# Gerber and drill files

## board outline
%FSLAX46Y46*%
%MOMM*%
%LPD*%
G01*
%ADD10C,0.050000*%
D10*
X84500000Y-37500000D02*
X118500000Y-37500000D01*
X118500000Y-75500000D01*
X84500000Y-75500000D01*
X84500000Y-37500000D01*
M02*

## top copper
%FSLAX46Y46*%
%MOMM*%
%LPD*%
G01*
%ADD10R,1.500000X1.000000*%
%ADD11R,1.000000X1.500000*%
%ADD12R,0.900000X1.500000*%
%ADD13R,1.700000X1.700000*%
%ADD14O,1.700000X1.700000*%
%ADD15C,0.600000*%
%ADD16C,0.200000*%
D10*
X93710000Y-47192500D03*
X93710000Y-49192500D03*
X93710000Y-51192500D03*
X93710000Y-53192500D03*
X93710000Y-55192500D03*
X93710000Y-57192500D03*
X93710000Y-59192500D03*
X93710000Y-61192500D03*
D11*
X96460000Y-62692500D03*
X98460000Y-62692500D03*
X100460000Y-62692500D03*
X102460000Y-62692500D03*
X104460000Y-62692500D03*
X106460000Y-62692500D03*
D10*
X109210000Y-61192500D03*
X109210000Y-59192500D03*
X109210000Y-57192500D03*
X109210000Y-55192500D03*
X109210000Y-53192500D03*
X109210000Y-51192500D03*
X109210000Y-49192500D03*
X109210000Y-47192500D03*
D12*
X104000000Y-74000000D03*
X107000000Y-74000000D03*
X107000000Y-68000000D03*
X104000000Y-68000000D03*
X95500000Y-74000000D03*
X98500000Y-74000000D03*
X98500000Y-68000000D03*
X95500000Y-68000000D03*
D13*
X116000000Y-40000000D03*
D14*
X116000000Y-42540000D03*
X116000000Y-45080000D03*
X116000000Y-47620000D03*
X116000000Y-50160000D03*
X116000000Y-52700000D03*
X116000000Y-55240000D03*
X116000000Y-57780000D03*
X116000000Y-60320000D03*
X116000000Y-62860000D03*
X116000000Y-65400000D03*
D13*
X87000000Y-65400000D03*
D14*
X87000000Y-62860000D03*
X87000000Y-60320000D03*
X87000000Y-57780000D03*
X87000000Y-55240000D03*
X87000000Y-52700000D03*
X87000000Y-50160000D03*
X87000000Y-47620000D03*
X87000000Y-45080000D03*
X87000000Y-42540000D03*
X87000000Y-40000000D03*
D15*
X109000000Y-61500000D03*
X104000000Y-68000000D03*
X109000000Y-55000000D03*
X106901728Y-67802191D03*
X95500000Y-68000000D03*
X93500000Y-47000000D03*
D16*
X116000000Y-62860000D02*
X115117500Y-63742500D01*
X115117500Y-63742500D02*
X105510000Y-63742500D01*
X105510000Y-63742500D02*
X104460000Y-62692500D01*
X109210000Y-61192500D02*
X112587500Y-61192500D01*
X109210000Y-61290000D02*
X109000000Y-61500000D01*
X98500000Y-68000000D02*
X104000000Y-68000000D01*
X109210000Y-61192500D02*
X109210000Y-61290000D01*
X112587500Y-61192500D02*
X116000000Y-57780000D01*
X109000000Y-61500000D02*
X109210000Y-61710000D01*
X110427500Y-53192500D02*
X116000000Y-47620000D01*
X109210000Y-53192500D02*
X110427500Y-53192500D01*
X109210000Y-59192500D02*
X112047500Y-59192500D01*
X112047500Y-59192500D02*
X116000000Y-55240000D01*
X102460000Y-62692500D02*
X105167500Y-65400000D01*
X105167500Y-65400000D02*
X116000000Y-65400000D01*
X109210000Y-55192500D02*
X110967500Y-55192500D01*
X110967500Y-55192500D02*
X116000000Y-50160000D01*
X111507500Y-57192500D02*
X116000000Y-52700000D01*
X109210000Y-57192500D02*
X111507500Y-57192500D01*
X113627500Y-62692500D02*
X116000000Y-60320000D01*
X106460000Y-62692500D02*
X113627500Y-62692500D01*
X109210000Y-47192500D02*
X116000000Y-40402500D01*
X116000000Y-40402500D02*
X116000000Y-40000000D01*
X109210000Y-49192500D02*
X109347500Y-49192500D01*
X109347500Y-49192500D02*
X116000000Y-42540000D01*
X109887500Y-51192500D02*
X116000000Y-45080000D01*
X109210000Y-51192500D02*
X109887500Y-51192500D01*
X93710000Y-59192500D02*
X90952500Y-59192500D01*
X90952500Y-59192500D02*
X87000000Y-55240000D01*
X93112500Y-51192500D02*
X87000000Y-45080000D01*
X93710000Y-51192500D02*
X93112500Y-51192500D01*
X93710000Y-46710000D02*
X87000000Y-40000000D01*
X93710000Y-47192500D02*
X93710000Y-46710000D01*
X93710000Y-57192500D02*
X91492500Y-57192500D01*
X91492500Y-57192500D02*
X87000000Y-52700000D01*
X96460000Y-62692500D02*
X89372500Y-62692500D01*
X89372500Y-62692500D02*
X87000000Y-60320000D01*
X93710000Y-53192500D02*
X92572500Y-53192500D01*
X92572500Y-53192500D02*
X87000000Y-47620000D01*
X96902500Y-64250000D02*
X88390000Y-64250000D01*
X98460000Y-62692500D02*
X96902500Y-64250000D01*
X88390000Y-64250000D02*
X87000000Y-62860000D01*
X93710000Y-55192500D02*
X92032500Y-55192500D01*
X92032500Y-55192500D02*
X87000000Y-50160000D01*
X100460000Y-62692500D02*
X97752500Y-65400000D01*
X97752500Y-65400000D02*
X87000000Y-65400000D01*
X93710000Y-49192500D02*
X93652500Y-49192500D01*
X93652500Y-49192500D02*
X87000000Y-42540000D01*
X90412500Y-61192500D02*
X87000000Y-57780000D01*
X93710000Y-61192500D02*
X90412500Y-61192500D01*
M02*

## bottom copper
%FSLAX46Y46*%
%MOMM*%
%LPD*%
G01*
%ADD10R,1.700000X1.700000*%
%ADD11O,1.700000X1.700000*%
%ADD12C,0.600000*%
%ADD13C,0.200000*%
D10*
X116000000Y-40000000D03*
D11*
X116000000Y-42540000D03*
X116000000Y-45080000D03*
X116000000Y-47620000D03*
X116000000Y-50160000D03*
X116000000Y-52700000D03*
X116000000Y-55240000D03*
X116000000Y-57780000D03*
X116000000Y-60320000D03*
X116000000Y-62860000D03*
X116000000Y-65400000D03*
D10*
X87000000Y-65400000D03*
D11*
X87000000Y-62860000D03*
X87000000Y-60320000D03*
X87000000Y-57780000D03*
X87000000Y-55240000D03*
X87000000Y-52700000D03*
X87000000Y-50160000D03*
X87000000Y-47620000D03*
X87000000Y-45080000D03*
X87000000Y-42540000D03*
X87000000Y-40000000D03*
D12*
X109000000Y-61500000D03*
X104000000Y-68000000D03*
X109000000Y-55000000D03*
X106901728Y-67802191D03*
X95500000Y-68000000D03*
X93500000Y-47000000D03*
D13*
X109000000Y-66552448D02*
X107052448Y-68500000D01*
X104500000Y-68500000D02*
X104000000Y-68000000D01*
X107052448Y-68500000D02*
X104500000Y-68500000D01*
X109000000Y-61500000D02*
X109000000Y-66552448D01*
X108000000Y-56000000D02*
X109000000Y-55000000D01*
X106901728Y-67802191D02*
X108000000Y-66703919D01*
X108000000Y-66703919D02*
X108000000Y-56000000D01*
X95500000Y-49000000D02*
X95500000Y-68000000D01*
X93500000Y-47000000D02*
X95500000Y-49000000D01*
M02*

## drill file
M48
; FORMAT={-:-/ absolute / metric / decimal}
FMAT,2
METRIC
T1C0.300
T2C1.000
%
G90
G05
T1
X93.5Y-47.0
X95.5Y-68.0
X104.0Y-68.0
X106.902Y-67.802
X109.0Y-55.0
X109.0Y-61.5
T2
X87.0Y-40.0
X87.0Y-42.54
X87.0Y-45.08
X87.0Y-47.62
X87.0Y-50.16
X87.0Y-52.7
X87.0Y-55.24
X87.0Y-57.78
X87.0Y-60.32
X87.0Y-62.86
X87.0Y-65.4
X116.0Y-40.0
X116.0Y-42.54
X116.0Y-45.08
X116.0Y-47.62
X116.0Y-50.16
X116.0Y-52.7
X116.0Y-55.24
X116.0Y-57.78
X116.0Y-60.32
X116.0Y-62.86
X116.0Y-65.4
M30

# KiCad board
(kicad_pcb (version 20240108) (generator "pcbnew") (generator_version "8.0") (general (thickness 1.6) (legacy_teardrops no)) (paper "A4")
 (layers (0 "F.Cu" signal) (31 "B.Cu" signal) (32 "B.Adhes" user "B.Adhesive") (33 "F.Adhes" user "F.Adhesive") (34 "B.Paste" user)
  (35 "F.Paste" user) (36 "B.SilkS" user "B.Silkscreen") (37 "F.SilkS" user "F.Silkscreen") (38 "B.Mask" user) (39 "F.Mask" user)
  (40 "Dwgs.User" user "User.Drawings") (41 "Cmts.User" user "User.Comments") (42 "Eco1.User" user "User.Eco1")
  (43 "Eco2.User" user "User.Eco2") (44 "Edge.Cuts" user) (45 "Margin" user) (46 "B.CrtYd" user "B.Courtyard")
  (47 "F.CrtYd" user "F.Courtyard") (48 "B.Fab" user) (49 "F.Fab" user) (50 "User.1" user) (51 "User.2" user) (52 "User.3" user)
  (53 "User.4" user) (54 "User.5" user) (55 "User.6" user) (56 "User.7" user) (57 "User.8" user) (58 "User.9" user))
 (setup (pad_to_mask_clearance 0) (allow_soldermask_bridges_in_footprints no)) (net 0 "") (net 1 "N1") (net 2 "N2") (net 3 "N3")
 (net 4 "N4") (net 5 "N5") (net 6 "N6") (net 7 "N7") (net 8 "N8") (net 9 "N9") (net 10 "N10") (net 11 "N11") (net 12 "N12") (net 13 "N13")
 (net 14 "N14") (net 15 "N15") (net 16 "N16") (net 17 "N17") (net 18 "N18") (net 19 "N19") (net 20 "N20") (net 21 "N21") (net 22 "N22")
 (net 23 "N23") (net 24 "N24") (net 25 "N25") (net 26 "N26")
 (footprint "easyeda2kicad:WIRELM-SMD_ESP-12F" (layer "F.Cu") (at 101.46 54.9425)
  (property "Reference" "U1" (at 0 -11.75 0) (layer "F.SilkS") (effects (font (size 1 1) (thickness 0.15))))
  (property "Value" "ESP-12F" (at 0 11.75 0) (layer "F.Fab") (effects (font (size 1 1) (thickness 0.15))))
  (pad "1" smd rect (at -7.75 -7.75) (size 1.5 1) (layers "F.Cu" "F.Paste" "F.Mask") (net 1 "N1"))
  (pad "2" smd rect (at -7.75 -5.75) (size 1.5 1) (layers "F.Cu" "F.Paste" "F.Mask") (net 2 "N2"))
  (pad "3" smd rect (at -7.75 -3.75) (size 1.5 1) (layers "F.Cu" "F.Paste" "F.Mask") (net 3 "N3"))
  (pad "4" smd rect (at -7.75 -1.75) (size 1.5 1) (layers "F.Cu" "F.Paste" "F.Mask") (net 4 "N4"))
  (pad "5" smd rect (at -7.75 0.25) (size 1.5 1) (layers "F.Cu" "F.Paste" "F.Mask") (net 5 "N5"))
  (pad "6" smd rect (at -7.75 2.25) (size 1.5 1) (layers "F.Cu" "F.Paste" "F.Mask") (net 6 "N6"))
  (pad "7" smd rect (at -7.75 4.25) (size 1.5 1) (layers "F.Cu" "F.Paste" "F.Mask") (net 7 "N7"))
  (pad "8" smd rect (at -7.75 6.25) (size 1.5 1) (layers "F.Cu" "F.Paste" "F.Mask") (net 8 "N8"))
  (pad "9" smd rect (at -5 7.75 90) (size 1.5 1) (layers "F.Cu" "F.Paste" "F.Mask") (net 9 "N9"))
  (pad "10" smd rect (at -3 7.75 90) (size 1.5 1) (layers "F.Cu" "F.Paste" "F.Mask") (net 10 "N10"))
  (pad "11" smd rect (at -1 7.75 90) (size 1.5 1) (layers "F.Cu" "F.Paste" "F.Mask") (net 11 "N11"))
  (pad "12" smd rect (at 1 7.75 90) (size 1.5 1) (layers "F.Cu" "F.Paste" "F.Mask") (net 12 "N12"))
  (pad "13" smd rect (at 3 7.75 90) (size 1.5 1) (layers "F.Cu" "F.Paste" "F.Mask") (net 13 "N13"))
  (pad "14" smd rect (at 5 7.75 90) (size 1.5 1) (layers "F.Cu" "F.Paste" "F.Mask") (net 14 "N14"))
  (pad "15" smd rect (at 7.75 6.25 180) (size 1.5 1) (layers "F.Cu" "F.Paste" "F.Mask") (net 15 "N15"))
  (pad "16" smd rect (at 7.75 4.25 180) (size 1.5 1) (layers "F.Cu" "F.Paste" "F.Mask") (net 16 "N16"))
  (pad "17" smd rect (at 7.75 2.25 180) (size 1.5 1) (layers "F.Cu" "F.Paste" "F.Mask") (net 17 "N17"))
  (pad "18" smd rect (at 7.75 0.25 180) (size 1.5 1) (layers "F.Cu" "F.Paste" "F.Mask") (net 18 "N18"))
  (pad "19" smd rect (at 7.75 -1.75 180) (size 1.5 1) (layers "F.Cu" "F.Paste" "F.Mask") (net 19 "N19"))
  (pad "20" smd rect (at 7.75 -3.75 180) (size 1.5 1) (layers "F.Cu" "F.Paste" "F.Mask") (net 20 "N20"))
  (pad "21" smd rect (at 7.75 -5.75 180) (size 1.5 1) (layers "F.Cu" "F.Paste" "F.Mask") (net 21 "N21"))
  (pad "22" smd rect (at 7.75 -7.75 180) (size 1.5 1) (layers "F.Cu" "F.Paste" "F.Mask") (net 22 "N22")))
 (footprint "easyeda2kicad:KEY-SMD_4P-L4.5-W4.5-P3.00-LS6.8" (layer "F.Cu") (at 105.5 71 90)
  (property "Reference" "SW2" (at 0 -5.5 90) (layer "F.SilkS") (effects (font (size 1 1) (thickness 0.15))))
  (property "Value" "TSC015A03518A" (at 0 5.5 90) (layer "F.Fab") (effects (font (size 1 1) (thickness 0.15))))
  (pad "1" smd rect (at -3 -1.5 90) (size 1.5 0.9) (layers "F.Cu" "F.Paste" "F.Mask") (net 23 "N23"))
  (pad "2" smd rect (at -3 1.5 90) (size 1.5 0.9) (layers "F.Cu" "F.Paste" "F.Mask") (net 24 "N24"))
  (pad "3" smd rect (at 3 1.5 90) (size 1.5 0.9) (layers "F.Cu" "F.Paste" "F.Mask") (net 18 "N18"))
  (pad "4" smd rect (at 3 -1.5 90) (size 1.5 0.9) (layers "F.Cu" "F.Paste" "F.Mask") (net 15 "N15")))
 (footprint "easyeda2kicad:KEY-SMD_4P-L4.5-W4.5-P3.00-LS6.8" (layer "F.Cu") (at 97 71 90)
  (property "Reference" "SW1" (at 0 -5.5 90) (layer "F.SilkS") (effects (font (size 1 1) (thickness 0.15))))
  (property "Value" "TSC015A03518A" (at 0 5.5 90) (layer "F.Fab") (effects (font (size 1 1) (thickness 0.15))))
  (pad "1" smd rect (at -3 -1.5 90) (size 1.5 0.9) (layers "F.Cu" "F.Paste" "F.Mask") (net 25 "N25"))
  (pad "2" smd rect (at -3 1.5 90) (size 1.5 0.9) (layers "F.Cu" "F.Paste" "F.Mask") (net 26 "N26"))
  (pad "3" smd rect (at 3 1.5 90) (size 1.5 0.9) (layers "F.Cu" "F.Paste" "F.Mask") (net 15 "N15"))
  (pad "4" smd rect (at 3 -1.5 90) (size 1.5 0.9) (layers "F.Cu" "F.Paste" "F.Mask") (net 1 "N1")))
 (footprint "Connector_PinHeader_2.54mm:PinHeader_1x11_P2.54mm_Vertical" (layer "B.Cu") (at 116 40 180)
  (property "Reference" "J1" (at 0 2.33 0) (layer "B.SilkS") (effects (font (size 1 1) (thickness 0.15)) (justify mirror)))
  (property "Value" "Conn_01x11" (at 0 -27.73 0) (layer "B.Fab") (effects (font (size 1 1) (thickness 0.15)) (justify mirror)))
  (pad "1" thru_hole rect (at 0 0 180) (size 1.7 1.7) (drill 1) (layers "*.Cu" "*.Mask") (remove_unused_layers no) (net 22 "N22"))
  (pad "2" thru_hole oval (at 0 -2.54 180) (size 1.7 1.7) (drill 1) (layers "*.Cu" "*.Mask") (remove_unused_layers no) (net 21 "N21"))
  (pad "3" thru_hole oval (at 0 -5.08 180) (size 1.7 1.7) (drill 1) (layers "*.Cu" "*.Mask") (remove_unused_layers no) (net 20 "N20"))
  (pad "4" thru_hole oval (at 0 -7.62 180) (size 1.7 1.7) (drill 1) (layers "*.Cu" "*.Mask") (remove_unused_layers no) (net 19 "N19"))
  (pad "5" thru_hole oval (at 0 -10.16 180) (size 1.7 1.7) (drill 1) (layers "*.Cu" "*.Mask") (remove_unused_layers no) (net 18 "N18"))
  (pad "6" thru_hole oval (at 0 -12.7 180) (size 1.7 1.7) (drill 1) (layers "*.Cu" "*.Mask") (remove_unused_layers no) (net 17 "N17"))
  (pad "7" thru_hole oval (at 0 -15.24 180) (size 1.7 1.7) (drill 1) (layers "*.Cu" "*.Mask") (remove_unused_layers no) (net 16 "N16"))
  (pad "8" thru_hole oval (at 0 -17.78 180) (size 1.7 1.7) (drill 1) (layers "*.Cu" "*.Mask") (remove_unused_layers no) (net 15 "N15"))
  (pad "9" thru_hole oval (at 0 -20.32 180) (size 1.7 1.7) (drill 1) (layers "*.Cu" "*.Mask") (remove_unused_layers no) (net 14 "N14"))
  (pad "10" thru_hole oval (at 0 -22.86 180) (size 1.7 1.7) (drill 1) (layers "*.Cu" "*.Mask") (remove_unused_layers no) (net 13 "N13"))
  (pad "11" thru_hole oval (at 0 -25.4 180) (size 1.7 1.7) (drill 1) (layers "*.Cu" "*.Mask") (remove_unused_layers no) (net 12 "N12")))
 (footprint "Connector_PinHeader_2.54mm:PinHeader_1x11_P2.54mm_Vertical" (layer "B.Cu") (at 87 65.4)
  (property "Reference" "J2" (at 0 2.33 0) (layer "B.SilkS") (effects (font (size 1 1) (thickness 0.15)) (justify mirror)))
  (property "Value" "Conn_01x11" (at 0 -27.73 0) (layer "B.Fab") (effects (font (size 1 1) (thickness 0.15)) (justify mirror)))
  (pad "1" thru_hole rect (at 0 0) (size 1.7 1.7) (drill 1) (layers "*.Cu" "*.Mask") (remove_unused_layers no) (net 11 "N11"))
  (pad "2" thru_hole oval (at 0 -2.54) (size 1.7 1.7) (drill 1) (layers "*.Cu" "*.Mask") (remove_unused_layers no) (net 10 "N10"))
  (pad "3" thru_hole oval (at 0 -5.08) (size 1.7 1.7) (drill 1) (layers "*.Cu" "*.Mask") (remove_unused_layers no) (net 9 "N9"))
  (pad "4" thru_hole oval (at 0 -7.62) (size 1.7 1.7) (drill 1) (layers "*.Cu" "*.Mask") (remove_unused_layers no) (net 8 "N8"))
  (pad "5" thru_hole oval (at 0 -10.16) (size 1.7 1.7) (drill 1) (layers "*.Cu" "*.Mask") (remove_unused_layers no) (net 7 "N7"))
  (pad "6" thru_hole oval (at 0 -12.7) (size 1.7 1.7) (drill 1) (layers "*.Cu" "*.Mask") (remove_unused_layers no) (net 6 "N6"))
  (pad "7" thru_hole oval (at 0 -15.24) (size 1.7 1.7) (drill 1) (layers "*.Cu" "*.Mask") (remove_unused_layers no) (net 5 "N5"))
  (pad "8" thru_hole oval (at 0 -17.78) (size 1.7 1.7) (drill 1) (layers "*.Cu" "*.Mask") (remove_unused_layers no) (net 4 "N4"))
  (pad "9" thru_hole oval (at 0 -20.32) (size 1.7 1.7) (drill 1) (layers "*.Cu" "*.Mask") (remove_unused_layers no) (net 3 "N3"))
  (pad "10" thru_hole oval (at 0 -22.86) (size 1.7 1.7) (drill 1) (layers "*.Cu" "*.Mask") (remove_unused_layers no) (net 2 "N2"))
  (pad "11" thru_hole oval (at 0 -25.4) (size 1.7 1.7) (drill 1) (layers "*.Cu" "*.Mask") (remove_unused_layers no) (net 1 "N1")))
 (gr_rect (start 84.5 37.5) (end 118.5 75.5) (stroke (width 0.05) (type default)) (fill none) (layer "Edge.Cuts"))
 (segment (start 116 62.86) (end 115.1175 63.7425) (width 0.2) (layer "F.Cu") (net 13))
 (segment (start 115.1175 63.7425) (end 105.51 63.7425) (width 0.2) (layer "F.Cu") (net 13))
 (segment (start 105.51 63.7425) (end 104.46 62.6925) (width 0.2) (layer "F.Cu") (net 13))
 (segment (start 109.21 61.1925) (end 112.5875 61.1925) (width 0.2) (layer "F.Cu") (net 15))
 (segment (start 109.21 61.29) (end 109 61.5) (width 0.2) (layer "F.Cu") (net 15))
 (segment (start 98.5 68) (end 104 68) (width 0.2) (layer "F.Cu") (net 15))
 (segment (start 109.21 61.1925) (end 109.21 61.29) (width 0.2) (layer "F.Cu") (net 15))
 (segment (start 112.5875 61.1925) (end 116 57.78) (width 0.2) (layer "F.Cu") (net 15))
 (segment (start 109 61.5) (end 109.21 61.71) (width 0.2) (layer "F.Cu") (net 15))
 (via (at 109 61.5) (size 0.6) (drill 0.3) (layers "F.Cu" "B.Cu") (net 15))
 (via (at 104 68) (size 0.6) (drill 0.3) (layers "F.Cu" "B.Cu") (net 15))
 (segment (start 109 66.552448) (end 107.052448 68.5) (width 0.2) (layer "B.Cu") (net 15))
 (segment (start 104.5 68.5) (end 104 68) (width 0.2) (layer "B.Cu") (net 15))
 (segment (start 107.052448 68.5) (end 104.5 68.5) (width 0.2) (layer "B.Cu") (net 15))
 (segment (start 109 61.5) (end 109 66.552448) (width 0.2) (layer "B.Cu") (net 15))
 (segment (start 110.4275 53.1925) (end 116 47.62) (width 0.2) (layer "F.Cu") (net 19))
 (segment (start 109.21 53.1925) (end 110.4275 53.1925) (width 0.2) (layer "F.Cu") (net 19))
 (segment (start 109.21 59.1925) (end 112.0475 59.1925) (width 0.2) (layer "F.Cu") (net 16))
 (segment (start 112.0475 59.1925) (end 116 55.24) (width 0.2) (layer "F.Cu") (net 16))
 (segment (start 102.46 62.6925) (end 105.1675 65.4) (width 0.2) (layer "F.Cu") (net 12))
 (segment (start 105.1675 65.4) (end 116 65.4) (width 0.2) (layer "F.Cu") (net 12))
 (segment (start 109.21 55.1925) (end 110.9675 55.1925) (width 0.2) (layer "F.Cu") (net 18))
 (segment (start 110.9675 55.1925) (end 116 50.16) (width 0.2) (layer "F.Cu") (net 18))
 (via (at 109 55) (size 0.6) (drill 0.3) (layers "F.Cu" "B.Cu") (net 18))
 (via (at 106.901728 67.802191) (size 0.6) (drill 0.3) (layers "F.Cu" "B.Cu") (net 18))
 (segment (start 108 56) (end 109 55) (width 0.2) (layer "B.Cu") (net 18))
 (segment (start 106.901728 67.802191) (end 108 66.703919) (width 0.2) (layer "B.Cu") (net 18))
 (segment (start 108 66.703919) (end 108 56) (width 0.2) (layer "B.Cu") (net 18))
 (segment (start 111.5075 57.1925) (end 116 52.7) (width 0.2) (layer "F.Cu") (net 17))
 (segment (start 109.21 57.1925) (end 111.5075 57.1925) (width 0.2) (layer "F.Cu") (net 17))
 (segment (start 113.6275 62.6925) (end 116 60.32) (width 0.2) (layer "F.Cu") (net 14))
 (segment (start 106.46 62.6925) (end 113.6275 62.6925) (width 0.2) (layer "F.Cu") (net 14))
 (segment (start 109.21 47.1925) (end 116 40.4025) (width 0.2) (layer "F.Cu") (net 22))
 (segment (start 116 40.4025) (end 116 40) (width 0.2) (layer "F.Cu") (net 22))
 (segment (start 109.21 49.1925) (end 109.3475 49.1925) (width 0.2) (layer "F.Cu") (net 21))
 (segment (start 109.3475 49.1925) (end 116 42.54) (width 0.2) (layer "F.Cu") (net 21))
 (segment (start 109.8875 51.1925) (end 116 45.08) (width 0.2) (layer "F.Cu") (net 20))
 (segment (start 109.21 51.1925) (end 109.8875 51.1925) (width 0.2) (layer "F.Cu") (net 20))
 (segment (start 93.71 59.1925) (end 90.9525 59.1925) (width 0.2) (layer "F.Cu") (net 7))
 (segment (start 90.9525 59.1925) (end 87 55.24) (width 0.2) (layer "F.Cu") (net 7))
 (segment (start 93.1125 51.1925) (end 87 45.08) (width 0.2) (layer "F.Cu") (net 3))
 (segment (start 93.71 51.1925) (end 93.1125 51.1925) (width 0.2) (layer "F.Cu") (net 3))
 (segment (start 93.71 46.71) (end 87 40) (width 0.2) (layer "F.Cu") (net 1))
 (segment (start 93.71 47.1925) (end 93.71 46.71) (width 0.2) (layer "F.Cu") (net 1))
 (via (at 95.5 68) (size 0.6) (drill 0.3) (layers "F.Cu" "B.Cu") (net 1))
 (via (at 93.5 47) (size 0.6) (drill 0.3) (layers "F.Cu" "B.Cu") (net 1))
 (segment (start 95.5 49) (end 95.5 68) (width 0.2) (layer "B.Cu") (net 1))
 (segment (start 93.5 47) (end 95.5 49) (width 0.2) (layer "B.Cu") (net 1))
 (segment (start 93.71 57.1925) (end 91.4925 57.1925) (width 0.2) (layer "F.Cu") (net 6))
 (segment (start 91.4925 57.1925) (end 87 52.7) (width 0.2) (layer "F.Cu") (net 6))
 (segment (start 96.46 62.6925) (end 89.3725 62.6925) (width 0.2) (layer "F.Cu") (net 9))
 (segment (start 89.3725 62.6925) (end 87 60.32) (width 0.2) (layer "F.Cu") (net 9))
 (segment (start 93.71 53.1925) (end 92.5725 53.1925) (width 0.2) (layer "F.Cu") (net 4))
 (segment (start 92.5725 53.1925) (end 87 47.62) (width 0.2) (layer "F.Cu") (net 4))
 (segment (start 96.9025 64.25) (end 88.39 64.25) (width 0.2) (layer "F.Cu") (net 10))
 (segment (start 98.46 62.6925) (end 96.9025 64.25) (width 0.2) (layer "F.Cu") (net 10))
 (segment (start 88.39 64.25) (end 87 62.86) (width 0.2) (layer "F.Cu") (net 10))
 (segment (start 93.71 55.1925) (end 92.0325 55.1925) (width 0.2) (layer "F.Cu") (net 5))
 (segment (start 92.0325 55.1925) (end 87 50.16) (width 0.2) (layer "F.Cu") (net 5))
 (segment (start 100.46 62.6925) (end 97.7525 65.4) (width 0.2) (layer "F.Cu") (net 11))
 (segment (start 97.7525 65.4) (end 87 65.4) (width 0.2) (layer "F.Cu") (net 11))
 (segment (start 93.71 49.1925) (end 93.6525 49.1925) (width 0.2) (layer "F.Cu") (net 2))
 (segment (start 93.6525 49.1925) (end 87 42.54) (width 0.2) (layer "F.Cu") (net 2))
 (segment (start 90.4125 61.1925) (end 87 57.78) (width 0.2) (layer "F.Cu") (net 8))
 (segment (start 93.71 61.1925) (end 90.4125 61.1925) (width 0.2) (layer "F.Cu") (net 8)))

